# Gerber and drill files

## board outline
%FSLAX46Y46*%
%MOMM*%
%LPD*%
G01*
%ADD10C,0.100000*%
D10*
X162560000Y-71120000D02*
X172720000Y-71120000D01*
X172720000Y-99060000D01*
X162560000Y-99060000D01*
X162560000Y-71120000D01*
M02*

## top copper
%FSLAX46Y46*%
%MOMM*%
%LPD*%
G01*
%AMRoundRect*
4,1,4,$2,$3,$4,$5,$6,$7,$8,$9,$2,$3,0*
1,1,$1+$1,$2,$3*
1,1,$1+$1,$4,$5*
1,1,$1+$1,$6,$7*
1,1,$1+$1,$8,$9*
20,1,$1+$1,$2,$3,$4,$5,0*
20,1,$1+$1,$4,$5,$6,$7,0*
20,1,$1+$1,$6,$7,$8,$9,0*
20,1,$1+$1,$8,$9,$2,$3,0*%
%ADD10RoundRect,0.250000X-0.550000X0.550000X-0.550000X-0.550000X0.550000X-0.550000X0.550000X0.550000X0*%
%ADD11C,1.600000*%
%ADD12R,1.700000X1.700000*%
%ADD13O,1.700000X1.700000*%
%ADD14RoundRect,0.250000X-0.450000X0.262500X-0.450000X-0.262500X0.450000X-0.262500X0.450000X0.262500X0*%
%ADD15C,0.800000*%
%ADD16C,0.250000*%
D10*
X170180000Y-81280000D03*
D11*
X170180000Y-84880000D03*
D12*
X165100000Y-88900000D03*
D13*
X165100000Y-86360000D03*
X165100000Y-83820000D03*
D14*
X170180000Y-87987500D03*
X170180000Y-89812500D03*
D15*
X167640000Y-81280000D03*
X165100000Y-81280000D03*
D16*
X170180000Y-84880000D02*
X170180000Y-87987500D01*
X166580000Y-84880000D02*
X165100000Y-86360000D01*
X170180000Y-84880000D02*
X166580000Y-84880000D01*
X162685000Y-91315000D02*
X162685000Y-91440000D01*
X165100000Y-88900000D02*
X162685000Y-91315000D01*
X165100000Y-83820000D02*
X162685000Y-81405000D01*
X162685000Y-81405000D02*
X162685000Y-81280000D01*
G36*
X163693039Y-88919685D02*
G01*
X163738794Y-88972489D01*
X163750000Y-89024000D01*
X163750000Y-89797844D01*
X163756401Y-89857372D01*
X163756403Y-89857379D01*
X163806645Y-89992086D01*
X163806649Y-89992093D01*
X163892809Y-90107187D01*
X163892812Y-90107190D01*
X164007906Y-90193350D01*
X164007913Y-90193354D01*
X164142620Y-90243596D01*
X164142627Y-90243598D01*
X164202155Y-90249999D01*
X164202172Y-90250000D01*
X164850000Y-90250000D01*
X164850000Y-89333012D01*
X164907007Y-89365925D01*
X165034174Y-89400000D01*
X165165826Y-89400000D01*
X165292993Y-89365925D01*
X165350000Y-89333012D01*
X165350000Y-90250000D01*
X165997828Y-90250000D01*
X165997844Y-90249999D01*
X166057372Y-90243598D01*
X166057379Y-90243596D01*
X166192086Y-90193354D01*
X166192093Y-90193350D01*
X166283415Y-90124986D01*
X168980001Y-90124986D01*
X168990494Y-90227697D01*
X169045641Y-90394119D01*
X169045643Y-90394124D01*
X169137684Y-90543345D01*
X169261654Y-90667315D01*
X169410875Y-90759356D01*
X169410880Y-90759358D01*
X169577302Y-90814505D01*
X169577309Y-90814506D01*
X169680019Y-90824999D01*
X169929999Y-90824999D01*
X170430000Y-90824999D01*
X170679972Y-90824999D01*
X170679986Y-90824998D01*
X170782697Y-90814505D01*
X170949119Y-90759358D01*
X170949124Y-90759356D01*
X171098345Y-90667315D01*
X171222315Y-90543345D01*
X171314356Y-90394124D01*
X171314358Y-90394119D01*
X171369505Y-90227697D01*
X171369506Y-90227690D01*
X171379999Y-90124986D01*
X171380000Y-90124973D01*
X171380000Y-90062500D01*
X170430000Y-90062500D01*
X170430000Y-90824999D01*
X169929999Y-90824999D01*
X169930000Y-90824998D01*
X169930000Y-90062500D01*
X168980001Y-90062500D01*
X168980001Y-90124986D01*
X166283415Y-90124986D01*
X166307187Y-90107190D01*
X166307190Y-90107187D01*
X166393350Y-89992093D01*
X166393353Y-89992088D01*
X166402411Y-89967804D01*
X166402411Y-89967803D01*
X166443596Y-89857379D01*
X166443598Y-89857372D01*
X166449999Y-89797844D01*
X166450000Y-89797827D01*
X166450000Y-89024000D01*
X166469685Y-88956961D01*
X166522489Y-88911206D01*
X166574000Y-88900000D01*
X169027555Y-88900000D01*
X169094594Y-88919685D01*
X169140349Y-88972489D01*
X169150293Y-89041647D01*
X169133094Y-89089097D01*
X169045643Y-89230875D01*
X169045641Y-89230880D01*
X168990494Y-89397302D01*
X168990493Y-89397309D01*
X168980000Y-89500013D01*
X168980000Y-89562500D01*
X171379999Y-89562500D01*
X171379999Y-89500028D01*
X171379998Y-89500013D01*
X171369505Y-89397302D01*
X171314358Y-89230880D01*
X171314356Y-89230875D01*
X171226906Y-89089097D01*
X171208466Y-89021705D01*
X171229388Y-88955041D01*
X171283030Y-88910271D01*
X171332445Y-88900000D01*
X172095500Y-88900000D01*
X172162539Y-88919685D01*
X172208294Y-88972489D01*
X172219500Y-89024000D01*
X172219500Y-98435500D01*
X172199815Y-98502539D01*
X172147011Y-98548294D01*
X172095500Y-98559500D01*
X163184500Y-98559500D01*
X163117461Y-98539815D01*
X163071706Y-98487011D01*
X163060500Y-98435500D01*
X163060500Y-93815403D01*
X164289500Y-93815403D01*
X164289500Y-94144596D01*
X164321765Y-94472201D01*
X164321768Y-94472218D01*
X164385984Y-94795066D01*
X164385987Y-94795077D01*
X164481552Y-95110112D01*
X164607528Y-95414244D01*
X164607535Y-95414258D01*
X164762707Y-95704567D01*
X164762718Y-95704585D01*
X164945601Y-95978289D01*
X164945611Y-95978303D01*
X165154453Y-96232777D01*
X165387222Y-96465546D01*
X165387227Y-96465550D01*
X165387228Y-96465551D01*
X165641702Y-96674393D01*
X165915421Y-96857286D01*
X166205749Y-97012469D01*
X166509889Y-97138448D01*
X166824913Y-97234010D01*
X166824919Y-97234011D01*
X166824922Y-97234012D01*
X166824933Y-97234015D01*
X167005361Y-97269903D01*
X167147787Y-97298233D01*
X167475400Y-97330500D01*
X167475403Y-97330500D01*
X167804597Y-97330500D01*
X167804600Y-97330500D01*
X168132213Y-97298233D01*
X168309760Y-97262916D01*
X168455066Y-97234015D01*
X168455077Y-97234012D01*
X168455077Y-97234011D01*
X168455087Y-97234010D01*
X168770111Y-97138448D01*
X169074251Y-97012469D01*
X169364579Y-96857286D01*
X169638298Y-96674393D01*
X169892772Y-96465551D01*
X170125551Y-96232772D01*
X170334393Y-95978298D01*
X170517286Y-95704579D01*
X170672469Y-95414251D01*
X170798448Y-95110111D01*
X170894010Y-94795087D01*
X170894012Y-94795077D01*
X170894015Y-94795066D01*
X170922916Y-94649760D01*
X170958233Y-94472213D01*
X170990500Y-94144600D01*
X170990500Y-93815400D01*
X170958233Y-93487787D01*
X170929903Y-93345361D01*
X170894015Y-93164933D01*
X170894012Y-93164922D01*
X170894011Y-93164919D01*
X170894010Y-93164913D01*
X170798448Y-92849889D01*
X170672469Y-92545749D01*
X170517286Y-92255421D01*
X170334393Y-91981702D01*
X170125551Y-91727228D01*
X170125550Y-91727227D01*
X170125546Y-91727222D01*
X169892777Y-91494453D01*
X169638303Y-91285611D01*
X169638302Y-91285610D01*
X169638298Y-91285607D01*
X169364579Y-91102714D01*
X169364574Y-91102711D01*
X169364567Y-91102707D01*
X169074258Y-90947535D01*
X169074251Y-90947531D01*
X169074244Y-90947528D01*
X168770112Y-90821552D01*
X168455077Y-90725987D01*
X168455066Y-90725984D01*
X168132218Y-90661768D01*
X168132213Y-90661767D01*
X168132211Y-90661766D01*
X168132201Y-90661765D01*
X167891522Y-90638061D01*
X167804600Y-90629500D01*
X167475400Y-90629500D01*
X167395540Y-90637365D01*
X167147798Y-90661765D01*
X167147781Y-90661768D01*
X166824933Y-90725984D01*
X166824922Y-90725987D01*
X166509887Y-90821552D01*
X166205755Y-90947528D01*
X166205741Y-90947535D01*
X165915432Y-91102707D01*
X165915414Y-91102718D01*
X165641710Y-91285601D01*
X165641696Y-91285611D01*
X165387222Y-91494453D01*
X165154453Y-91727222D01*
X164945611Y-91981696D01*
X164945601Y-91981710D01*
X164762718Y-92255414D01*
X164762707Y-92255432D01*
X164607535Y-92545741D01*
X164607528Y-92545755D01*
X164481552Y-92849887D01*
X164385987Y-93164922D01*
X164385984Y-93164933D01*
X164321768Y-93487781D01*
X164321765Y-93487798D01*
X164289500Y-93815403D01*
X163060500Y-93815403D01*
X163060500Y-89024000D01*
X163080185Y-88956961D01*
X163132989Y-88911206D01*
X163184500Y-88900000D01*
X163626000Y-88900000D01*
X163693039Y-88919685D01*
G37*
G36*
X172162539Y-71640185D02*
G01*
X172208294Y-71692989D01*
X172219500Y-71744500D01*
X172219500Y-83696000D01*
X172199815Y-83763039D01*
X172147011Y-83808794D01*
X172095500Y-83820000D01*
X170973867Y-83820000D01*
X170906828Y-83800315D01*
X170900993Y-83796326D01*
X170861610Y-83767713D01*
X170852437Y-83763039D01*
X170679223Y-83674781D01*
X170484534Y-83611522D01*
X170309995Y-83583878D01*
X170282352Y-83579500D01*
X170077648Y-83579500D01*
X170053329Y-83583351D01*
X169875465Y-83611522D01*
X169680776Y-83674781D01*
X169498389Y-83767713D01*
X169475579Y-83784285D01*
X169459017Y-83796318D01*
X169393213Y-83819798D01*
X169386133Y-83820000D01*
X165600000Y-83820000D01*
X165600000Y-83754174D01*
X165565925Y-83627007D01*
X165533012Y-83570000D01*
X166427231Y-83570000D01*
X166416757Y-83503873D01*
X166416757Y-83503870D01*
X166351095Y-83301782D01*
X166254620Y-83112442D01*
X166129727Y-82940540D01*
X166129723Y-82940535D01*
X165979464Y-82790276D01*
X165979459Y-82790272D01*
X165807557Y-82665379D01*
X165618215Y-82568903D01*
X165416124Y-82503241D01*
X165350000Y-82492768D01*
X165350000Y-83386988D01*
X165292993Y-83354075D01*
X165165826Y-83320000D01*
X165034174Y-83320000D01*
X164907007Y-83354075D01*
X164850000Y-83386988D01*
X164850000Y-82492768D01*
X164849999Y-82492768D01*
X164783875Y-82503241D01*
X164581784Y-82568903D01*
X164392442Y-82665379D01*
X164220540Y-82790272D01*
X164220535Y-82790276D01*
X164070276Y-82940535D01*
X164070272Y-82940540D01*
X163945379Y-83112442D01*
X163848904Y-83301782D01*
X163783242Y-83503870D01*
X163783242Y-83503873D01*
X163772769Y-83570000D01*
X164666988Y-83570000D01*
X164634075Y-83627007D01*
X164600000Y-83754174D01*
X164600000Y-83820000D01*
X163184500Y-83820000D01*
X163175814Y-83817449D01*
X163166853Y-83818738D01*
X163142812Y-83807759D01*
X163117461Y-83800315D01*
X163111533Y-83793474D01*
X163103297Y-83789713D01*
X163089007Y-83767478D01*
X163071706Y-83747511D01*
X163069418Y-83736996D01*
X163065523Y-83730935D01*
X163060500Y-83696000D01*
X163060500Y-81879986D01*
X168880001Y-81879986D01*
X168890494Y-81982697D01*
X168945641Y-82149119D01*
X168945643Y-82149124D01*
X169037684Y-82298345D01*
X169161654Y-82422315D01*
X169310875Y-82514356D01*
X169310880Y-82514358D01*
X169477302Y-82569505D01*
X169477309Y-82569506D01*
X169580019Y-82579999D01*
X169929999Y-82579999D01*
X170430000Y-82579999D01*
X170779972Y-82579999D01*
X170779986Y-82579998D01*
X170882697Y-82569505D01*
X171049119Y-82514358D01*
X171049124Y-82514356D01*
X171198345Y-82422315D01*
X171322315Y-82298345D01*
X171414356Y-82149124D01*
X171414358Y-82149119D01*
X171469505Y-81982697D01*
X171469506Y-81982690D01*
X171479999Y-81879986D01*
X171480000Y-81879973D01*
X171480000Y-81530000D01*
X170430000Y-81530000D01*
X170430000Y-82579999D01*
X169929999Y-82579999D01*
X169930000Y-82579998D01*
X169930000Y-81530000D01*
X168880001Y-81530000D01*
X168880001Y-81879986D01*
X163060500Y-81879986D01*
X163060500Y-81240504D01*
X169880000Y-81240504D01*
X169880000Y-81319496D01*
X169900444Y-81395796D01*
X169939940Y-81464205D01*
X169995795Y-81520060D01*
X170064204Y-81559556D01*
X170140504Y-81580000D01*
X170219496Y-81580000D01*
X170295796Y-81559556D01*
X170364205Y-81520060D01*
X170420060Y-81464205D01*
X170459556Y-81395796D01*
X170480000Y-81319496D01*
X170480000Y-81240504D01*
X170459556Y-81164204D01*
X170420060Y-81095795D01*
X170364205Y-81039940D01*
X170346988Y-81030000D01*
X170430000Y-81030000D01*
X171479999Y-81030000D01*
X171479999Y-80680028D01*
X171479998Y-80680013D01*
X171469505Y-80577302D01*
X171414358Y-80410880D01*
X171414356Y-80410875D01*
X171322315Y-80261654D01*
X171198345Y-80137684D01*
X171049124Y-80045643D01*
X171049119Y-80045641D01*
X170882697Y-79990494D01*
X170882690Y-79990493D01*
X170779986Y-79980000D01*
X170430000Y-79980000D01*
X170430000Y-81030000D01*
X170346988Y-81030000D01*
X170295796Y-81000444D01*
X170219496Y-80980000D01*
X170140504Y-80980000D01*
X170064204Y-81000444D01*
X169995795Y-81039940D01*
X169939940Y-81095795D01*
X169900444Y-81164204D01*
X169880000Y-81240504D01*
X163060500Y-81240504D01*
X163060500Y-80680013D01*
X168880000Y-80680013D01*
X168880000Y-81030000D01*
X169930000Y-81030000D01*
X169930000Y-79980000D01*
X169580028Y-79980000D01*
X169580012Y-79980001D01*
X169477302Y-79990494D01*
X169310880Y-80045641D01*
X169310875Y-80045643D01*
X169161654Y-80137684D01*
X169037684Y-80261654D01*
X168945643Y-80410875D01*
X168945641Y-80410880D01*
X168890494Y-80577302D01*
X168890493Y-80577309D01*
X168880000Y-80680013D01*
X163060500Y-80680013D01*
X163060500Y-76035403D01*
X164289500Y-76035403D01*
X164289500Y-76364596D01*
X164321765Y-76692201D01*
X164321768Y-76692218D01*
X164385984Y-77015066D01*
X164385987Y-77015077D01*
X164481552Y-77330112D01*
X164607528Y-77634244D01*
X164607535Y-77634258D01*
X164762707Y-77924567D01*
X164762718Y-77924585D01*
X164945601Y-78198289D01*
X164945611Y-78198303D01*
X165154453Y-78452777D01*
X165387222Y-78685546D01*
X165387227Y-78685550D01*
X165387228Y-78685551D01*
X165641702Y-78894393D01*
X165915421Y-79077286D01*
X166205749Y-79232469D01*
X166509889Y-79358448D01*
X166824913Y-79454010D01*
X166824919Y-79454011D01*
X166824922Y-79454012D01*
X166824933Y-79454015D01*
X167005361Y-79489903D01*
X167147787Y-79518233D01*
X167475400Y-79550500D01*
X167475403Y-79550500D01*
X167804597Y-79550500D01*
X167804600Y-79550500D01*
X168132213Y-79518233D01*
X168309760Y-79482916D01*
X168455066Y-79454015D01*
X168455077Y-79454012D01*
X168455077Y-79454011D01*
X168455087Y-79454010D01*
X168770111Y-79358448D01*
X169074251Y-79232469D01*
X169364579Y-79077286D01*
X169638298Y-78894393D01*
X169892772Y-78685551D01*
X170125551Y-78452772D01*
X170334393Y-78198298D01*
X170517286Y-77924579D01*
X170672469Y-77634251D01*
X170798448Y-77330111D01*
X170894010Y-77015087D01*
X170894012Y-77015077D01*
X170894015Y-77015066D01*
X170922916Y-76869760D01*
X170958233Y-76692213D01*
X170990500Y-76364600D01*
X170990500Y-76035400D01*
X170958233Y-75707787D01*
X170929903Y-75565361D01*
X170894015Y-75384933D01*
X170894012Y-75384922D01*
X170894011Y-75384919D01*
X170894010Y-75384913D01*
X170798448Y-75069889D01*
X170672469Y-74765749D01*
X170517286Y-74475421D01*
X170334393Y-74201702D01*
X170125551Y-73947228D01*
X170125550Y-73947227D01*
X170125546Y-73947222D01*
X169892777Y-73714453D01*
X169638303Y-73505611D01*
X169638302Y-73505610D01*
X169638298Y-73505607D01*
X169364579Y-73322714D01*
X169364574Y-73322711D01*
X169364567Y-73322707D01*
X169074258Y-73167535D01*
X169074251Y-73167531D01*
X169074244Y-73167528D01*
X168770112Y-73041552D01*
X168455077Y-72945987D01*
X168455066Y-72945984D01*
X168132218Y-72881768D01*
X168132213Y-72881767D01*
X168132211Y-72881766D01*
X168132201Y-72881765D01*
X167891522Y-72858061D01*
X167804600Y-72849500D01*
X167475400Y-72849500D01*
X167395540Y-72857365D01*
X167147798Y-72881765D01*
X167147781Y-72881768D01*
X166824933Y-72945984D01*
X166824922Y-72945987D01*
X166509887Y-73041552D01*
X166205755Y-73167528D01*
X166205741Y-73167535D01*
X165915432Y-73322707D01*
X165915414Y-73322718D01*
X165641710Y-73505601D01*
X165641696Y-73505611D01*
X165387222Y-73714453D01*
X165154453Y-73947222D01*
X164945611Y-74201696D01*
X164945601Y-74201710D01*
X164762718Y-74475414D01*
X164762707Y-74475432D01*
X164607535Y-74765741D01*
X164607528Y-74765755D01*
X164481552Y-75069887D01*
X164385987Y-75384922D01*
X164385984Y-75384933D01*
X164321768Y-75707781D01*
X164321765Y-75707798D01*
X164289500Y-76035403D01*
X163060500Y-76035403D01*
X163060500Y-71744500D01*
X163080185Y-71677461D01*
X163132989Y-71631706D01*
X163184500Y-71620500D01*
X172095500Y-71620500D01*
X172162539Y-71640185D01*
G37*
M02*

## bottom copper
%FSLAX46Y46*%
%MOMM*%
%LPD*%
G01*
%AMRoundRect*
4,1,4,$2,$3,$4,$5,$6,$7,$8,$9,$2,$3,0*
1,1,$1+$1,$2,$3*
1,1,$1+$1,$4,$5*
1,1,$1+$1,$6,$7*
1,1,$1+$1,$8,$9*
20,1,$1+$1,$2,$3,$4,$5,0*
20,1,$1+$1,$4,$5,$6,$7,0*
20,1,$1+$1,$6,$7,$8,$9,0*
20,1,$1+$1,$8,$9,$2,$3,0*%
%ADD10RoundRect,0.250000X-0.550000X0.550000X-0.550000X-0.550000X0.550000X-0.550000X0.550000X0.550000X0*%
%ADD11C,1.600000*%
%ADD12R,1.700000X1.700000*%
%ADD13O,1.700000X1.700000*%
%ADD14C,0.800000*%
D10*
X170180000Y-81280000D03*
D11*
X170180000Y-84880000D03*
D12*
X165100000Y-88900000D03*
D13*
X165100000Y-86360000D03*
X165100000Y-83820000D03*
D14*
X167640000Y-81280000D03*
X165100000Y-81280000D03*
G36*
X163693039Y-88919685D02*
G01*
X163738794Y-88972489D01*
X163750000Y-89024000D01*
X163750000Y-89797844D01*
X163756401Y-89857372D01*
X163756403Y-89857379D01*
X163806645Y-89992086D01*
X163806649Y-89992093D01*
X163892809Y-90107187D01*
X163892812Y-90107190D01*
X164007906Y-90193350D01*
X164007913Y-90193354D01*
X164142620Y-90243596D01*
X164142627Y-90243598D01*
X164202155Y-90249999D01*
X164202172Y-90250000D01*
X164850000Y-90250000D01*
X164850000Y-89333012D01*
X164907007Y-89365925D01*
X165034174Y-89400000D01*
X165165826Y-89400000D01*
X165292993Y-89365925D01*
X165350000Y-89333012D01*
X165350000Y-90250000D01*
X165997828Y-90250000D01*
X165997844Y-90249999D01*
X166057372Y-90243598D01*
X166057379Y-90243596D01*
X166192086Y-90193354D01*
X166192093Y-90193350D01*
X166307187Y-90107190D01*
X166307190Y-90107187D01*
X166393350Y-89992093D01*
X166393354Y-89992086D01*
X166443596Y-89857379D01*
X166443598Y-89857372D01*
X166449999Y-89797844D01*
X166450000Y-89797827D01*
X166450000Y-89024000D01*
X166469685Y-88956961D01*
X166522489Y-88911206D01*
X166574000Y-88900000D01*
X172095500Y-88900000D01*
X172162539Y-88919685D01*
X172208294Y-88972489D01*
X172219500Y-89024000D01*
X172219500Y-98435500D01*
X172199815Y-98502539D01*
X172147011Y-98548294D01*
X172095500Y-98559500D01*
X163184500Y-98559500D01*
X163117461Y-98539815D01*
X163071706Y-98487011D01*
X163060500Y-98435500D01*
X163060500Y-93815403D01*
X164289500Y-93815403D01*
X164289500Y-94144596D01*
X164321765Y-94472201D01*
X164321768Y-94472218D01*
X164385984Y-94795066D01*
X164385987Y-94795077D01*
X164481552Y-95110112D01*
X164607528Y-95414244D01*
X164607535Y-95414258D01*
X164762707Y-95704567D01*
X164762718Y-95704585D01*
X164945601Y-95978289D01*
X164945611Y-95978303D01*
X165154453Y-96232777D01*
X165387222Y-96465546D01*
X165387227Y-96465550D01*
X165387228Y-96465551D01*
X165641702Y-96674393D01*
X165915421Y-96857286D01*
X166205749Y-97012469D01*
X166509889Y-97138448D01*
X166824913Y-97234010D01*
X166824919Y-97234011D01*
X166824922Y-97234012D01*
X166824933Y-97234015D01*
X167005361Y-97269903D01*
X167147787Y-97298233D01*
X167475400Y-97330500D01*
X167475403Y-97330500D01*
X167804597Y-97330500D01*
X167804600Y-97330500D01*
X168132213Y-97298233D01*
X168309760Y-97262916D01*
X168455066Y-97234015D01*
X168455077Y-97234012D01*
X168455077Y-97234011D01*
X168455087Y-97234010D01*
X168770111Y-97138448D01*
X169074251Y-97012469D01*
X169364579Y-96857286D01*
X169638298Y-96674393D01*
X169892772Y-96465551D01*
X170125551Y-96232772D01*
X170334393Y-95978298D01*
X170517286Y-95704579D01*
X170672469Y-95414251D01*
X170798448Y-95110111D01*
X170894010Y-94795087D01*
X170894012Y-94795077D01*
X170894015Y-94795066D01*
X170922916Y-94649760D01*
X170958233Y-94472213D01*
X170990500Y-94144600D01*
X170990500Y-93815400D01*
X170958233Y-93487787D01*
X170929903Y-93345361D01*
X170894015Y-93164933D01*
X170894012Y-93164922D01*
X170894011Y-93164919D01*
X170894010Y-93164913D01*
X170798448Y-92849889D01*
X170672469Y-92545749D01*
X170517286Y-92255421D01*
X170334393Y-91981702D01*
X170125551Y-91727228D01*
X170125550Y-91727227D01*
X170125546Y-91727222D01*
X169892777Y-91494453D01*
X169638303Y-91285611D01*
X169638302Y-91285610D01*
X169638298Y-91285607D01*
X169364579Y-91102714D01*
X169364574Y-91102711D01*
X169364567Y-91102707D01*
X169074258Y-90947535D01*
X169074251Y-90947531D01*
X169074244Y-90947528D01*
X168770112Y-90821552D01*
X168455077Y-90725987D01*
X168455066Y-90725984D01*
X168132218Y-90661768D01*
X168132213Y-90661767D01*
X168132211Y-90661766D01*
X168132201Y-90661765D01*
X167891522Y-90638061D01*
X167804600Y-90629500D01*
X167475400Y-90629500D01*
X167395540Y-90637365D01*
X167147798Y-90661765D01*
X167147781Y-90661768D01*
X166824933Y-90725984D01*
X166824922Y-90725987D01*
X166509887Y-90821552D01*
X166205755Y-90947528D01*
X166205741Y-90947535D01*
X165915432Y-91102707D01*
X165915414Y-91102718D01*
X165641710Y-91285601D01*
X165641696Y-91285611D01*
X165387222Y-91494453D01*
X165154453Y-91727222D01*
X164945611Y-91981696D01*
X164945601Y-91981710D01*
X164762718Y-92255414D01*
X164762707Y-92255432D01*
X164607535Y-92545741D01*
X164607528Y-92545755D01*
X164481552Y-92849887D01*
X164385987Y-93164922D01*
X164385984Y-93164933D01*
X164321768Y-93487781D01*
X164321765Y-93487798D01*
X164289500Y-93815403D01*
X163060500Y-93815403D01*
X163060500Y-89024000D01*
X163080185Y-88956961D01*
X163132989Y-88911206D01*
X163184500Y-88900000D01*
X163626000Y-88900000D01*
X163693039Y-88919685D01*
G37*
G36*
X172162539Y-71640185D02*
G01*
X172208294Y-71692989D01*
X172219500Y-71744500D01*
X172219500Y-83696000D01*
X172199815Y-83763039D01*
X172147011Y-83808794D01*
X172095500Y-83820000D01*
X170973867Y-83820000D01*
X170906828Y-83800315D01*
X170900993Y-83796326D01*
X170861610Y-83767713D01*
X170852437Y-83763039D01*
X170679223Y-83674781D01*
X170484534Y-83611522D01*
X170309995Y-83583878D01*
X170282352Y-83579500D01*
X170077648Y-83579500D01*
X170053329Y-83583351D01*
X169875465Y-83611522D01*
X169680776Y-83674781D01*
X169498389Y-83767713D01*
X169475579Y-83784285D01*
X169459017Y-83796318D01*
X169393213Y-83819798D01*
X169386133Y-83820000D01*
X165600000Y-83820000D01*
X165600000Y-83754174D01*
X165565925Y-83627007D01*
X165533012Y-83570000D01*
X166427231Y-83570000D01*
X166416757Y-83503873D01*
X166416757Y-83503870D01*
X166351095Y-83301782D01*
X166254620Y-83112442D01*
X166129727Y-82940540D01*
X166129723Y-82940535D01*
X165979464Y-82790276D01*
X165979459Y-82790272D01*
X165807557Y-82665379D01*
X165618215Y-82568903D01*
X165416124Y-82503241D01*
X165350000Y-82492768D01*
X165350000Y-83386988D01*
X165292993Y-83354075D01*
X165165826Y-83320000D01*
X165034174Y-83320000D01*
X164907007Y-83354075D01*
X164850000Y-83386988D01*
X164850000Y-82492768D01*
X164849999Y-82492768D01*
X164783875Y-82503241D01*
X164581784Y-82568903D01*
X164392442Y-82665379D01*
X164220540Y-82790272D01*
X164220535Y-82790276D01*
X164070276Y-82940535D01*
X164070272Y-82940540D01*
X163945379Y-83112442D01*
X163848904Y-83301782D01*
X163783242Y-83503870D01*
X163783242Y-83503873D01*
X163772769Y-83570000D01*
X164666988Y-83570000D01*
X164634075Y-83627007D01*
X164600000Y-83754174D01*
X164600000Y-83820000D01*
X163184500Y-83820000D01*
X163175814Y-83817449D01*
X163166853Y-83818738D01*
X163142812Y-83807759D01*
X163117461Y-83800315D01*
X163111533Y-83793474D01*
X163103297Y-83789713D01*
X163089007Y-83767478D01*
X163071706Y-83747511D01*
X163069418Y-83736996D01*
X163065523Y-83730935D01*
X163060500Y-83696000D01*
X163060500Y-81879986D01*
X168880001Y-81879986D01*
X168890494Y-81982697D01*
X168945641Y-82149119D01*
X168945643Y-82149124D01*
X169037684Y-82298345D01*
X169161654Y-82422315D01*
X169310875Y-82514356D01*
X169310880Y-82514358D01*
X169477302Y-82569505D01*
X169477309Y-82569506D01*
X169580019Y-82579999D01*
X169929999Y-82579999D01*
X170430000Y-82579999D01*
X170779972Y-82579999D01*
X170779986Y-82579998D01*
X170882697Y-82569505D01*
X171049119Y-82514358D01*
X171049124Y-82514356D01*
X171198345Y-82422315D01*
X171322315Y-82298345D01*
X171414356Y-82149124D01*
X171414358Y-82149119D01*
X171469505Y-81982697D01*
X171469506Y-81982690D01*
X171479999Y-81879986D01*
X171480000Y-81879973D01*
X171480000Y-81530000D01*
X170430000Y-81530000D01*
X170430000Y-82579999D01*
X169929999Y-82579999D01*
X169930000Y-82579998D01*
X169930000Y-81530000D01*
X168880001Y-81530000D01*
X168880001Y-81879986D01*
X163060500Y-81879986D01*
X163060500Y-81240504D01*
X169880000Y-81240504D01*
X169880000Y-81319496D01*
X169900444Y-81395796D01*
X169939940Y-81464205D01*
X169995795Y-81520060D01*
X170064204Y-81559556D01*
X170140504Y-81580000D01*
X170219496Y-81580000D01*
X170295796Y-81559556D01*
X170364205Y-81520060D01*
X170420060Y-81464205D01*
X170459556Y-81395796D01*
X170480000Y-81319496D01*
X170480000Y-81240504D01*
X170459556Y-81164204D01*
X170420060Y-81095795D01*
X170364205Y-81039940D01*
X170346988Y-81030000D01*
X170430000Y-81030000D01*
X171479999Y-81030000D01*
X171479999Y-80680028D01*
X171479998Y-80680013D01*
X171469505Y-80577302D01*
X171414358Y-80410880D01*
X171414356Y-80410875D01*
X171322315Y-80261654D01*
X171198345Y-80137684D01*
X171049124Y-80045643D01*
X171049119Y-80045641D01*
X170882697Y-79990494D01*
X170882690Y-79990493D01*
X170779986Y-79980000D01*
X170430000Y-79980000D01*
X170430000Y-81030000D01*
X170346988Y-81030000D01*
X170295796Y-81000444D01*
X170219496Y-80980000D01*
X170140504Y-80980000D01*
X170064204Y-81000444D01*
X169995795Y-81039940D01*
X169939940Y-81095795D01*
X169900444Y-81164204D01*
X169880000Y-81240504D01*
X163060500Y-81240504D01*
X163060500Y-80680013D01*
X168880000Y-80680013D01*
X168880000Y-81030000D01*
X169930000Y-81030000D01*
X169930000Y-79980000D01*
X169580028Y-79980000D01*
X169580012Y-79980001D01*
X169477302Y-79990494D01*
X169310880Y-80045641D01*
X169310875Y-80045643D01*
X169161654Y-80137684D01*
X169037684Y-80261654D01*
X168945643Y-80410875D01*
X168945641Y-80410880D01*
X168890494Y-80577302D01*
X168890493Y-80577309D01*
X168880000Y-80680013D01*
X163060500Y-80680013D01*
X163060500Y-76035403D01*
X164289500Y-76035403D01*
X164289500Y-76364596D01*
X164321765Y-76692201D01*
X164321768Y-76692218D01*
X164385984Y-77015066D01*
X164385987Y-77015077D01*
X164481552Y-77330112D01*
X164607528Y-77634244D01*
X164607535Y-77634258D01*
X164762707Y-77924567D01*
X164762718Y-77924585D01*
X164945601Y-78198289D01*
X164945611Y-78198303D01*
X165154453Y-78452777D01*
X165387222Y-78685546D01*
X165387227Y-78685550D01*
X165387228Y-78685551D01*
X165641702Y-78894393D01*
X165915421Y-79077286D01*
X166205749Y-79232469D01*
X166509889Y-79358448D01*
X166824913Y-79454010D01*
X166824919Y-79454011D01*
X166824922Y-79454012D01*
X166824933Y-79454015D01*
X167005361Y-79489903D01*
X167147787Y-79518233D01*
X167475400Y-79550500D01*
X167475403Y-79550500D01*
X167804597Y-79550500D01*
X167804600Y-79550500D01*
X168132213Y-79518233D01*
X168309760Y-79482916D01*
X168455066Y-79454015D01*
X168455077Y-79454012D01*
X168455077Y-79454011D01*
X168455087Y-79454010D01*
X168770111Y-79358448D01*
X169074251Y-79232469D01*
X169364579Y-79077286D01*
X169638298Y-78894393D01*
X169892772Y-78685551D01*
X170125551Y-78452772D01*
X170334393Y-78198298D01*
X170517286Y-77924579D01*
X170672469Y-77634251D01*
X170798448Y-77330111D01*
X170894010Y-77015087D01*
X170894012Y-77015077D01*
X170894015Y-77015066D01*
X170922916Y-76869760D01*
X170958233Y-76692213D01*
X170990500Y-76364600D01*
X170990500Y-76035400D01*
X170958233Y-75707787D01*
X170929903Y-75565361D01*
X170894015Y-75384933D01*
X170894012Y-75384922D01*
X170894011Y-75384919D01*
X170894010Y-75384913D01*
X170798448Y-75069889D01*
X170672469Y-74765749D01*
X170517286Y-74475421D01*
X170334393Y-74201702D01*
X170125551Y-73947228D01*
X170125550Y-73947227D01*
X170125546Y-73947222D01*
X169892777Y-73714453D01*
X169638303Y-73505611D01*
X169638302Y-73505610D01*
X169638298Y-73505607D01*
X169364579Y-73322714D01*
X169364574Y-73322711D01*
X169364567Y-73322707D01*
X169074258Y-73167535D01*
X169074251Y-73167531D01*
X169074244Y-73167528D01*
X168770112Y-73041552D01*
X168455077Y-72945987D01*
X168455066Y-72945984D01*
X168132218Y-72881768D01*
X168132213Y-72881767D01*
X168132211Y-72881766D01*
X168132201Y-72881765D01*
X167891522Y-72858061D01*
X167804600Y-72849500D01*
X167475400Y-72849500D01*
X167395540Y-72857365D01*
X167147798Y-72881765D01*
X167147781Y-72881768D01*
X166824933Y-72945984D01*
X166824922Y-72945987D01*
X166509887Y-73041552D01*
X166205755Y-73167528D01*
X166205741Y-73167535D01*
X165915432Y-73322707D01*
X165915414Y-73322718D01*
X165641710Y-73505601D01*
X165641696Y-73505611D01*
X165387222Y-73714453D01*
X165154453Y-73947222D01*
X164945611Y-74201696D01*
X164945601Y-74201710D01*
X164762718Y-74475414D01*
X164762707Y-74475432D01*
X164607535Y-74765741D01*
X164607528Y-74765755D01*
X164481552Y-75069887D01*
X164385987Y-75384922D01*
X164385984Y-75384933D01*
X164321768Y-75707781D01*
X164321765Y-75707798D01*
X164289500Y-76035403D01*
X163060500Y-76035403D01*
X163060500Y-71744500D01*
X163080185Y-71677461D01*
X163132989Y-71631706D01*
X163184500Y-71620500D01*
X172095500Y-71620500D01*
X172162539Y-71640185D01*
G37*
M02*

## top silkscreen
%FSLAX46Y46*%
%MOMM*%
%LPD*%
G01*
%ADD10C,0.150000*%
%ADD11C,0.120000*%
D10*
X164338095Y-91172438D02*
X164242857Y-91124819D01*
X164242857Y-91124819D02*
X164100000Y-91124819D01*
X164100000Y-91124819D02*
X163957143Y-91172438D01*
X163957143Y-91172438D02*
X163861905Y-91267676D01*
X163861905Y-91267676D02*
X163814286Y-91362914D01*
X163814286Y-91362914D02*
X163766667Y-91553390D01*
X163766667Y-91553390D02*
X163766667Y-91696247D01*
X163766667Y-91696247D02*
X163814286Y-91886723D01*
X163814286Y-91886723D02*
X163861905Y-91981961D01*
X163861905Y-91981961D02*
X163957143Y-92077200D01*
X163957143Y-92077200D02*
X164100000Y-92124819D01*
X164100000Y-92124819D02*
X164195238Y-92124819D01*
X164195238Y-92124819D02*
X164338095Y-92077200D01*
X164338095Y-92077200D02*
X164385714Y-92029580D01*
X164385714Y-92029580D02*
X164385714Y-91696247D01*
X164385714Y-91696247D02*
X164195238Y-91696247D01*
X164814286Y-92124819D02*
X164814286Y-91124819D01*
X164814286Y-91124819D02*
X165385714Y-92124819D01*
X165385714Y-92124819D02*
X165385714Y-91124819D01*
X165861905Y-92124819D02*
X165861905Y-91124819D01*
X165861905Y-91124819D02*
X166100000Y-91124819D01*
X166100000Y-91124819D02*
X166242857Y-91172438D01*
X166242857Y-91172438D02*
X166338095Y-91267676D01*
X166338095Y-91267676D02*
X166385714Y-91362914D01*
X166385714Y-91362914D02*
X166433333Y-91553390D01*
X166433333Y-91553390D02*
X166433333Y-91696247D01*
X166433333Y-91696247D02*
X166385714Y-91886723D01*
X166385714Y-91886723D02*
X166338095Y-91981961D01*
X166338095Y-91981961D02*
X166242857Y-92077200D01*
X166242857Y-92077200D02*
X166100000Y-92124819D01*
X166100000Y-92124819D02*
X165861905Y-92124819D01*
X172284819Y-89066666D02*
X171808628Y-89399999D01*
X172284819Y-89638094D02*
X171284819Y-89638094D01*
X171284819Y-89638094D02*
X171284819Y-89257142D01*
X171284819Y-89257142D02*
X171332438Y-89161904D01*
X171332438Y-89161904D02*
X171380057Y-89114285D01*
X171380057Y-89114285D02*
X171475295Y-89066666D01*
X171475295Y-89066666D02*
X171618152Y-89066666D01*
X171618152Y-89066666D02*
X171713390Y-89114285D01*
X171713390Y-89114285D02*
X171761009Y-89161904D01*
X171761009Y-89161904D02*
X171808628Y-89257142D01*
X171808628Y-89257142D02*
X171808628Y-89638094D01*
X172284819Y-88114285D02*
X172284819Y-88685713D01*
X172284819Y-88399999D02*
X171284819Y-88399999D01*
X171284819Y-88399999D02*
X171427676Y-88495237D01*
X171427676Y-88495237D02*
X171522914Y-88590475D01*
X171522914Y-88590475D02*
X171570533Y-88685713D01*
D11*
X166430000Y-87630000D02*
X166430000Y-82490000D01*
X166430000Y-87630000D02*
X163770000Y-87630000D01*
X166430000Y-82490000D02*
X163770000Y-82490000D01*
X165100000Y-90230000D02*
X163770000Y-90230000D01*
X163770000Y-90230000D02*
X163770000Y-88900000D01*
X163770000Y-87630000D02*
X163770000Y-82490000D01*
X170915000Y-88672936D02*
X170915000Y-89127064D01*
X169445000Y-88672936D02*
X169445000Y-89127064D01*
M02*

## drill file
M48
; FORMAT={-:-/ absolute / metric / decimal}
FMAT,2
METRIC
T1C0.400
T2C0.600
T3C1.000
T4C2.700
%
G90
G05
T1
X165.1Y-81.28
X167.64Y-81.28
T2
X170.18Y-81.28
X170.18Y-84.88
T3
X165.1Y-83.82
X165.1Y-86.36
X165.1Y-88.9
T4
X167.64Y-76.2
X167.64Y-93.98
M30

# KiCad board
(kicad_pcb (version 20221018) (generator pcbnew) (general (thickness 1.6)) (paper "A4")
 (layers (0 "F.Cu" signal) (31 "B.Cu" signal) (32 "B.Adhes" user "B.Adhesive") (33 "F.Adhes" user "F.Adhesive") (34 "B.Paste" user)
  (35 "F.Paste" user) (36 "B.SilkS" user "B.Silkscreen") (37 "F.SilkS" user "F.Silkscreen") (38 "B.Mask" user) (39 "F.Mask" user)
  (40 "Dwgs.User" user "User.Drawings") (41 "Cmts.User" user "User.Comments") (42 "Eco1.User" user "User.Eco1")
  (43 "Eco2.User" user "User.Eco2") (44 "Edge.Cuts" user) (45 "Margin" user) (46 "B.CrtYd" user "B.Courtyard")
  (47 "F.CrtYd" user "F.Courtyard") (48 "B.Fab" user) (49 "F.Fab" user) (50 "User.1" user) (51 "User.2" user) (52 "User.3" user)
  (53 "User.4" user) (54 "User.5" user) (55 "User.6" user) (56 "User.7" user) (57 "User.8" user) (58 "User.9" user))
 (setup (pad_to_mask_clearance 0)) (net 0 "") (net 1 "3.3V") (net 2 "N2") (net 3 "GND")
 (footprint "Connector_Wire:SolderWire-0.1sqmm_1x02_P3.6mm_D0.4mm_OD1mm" (layer "F.Cu") (at 170.18 81.28 -90)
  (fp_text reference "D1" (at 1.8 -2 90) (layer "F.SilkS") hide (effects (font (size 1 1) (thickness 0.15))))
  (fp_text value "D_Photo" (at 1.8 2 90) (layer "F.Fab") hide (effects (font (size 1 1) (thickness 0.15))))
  (pad "1" thru_hole roundrect (at 0 0 270) (size 1.6 1.6) (drill 0.6) (layers "*.Cu" "*.Mask") (roundrect_rratio 0.15625) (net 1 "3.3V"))
  (pad "2" thru_hole circle (at 3.6 0 270) (size 1.6 1.6) (drill 0.6) (layers "*.Cu" "*.Mask") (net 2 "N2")))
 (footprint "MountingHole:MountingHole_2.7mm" (layer "F.Cu") (at 167.64 93.98)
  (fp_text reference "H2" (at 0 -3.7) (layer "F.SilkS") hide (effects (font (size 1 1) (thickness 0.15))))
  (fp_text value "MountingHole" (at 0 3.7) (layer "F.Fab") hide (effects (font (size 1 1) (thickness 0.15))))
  (pad "" np_thru_hole circle (at 0 0) (size 2.7 2.7) (drill 2.7) (layers "F&B.Cu" "*.Mask") (clearance 2)))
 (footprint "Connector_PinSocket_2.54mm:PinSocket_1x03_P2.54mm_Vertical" (layer "F.Cu") (at 165.1 88.9 180)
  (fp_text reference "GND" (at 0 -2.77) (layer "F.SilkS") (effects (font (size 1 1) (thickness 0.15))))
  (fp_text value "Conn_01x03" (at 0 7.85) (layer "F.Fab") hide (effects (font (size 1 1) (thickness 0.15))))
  (fp_line (start -1.33 1.27) (end -1.33 6.41) (stroke (width 0.12) (type solid)) (layer "F.SilkS"))
  (fp_line (start -1.33 1.27) (end 1.33 1.27) (stroke (width 0.12) (type solid)) (layer "F.SilkS"))
  (fp_line (start -1.33 6.41) (end 1.33 6.41) (stroke (width 0.12) (type solid)) (layer "F.SilkS"))
  (fp_line (start 0 -1.33) (end 1.33 -1.33) (stroke (width 0.12) (type solid)) (layer "F.SilkS"))
  (fp_line (start 1.33 -1.33) (end 1.33 0) (stroke (width 0.12) (type solid)) (layer "F.SilkS"))
  (fp_line (start 1.33 1.27) (end 1.33 6.41) (stroke (width 0.12) (type solid)) (layer "F.SilkS"))
  (pad "1" thru_hole rect (at 0 0 180) (size 1.7 1.7) (drill 1) (layers "*.Cu" "*.Mask") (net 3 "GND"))
  (pad "2" thru_hole oval (at 0 2.54 180) (size 1.7 1.7) (drill 1) (layers "*.Cu" "*.Mask") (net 2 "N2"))
  (pad "3" thru_hole oval (at 0 5.08 180) (size 1.7 1.7) (drill 1) (layers "*.Cu" "*.Mask") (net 1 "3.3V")))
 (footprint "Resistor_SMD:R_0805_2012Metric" (layer "F.Cu") (at 170.18 88.9 -90)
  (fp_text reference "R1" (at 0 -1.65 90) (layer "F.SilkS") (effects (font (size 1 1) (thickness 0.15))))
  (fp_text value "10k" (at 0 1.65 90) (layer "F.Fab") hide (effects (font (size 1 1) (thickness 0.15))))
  (fp_line (start -0.227064 -0.735) (end 0.227064 -0.735) (stroke (width 0.12) (type solid)) (layer "F.SilkS"))
  (fp_line (start -0.227064 0.735) (end 0.227064 0.735) (stroke (width 0.12) (type solid)) (layer "F.SilkS"))
  (pad "1" smd roundrect (at -0.9125 0 270) (size 1.025 1.4) (layers "F.Cu" "F.Paste" "F.Mask") (roundrect_rratio 0.243902) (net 2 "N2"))
  (pad "2" smd roundrect (at 0.9125 0 270) (size 1.025 1.4) (layers "F.Cu" "F.Paste" "F.Mask") (roundrect_rratio 0.243902) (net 3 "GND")))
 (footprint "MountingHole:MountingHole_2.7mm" (layer "F.Cu") (at 167.64 76.2)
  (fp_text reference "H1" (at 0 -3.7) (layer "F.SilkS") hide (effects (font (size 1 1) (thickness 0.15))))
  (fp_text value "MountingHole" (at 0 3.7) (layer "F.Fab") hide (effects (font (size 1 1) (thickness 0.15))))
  (pad "" np_thru_hole circle (at 0 0) (size 2.7 2.7) (drill 2.7) (layers "F&B.Cu" "*.Mask") (clearance 2)))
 (gr_rect (start 162.56 71.12) (end 172.72 99.06) (stroke (width 0.1) (type default)) (fill none) (layer "Edge.Cuts"))
 (segment (start 170.18 84.88) (end 170.18 87.9875) (width 0.25) (layer "F.Cu") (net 2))
 (segment (start 166.58 84.88) (end 165.1 86.36) (width 0.25) (layer "F.Cu") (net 2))
 (segment (start 170.18 84.88) (end 166.58 84.88) (width 0.25) (layer "F.Cu") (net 2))
 (segment (start 162.685 91.315) (end 162.685 91.44) (width 0.25) (layer "F.Cu") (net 3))
 (segment (start 165.1 88.9) (end 162.685 91.315) (width 0.25) (layer "F.Cu") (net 3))
 (segment (start 165.1 83.82) (end 162.685 81.405) (width 0.25) (layer "F.Cu") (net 1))
 (segment (start 162.685 81.405) (end 162.685 81.28) (width 0.25) (layer "F.Cu") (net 1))
 (via (at 167.64 81.28) (size 0.8) (drill 0.4) (layers "F.Cu" "B.Cu") (free) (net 1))
 (via (at 165.1 81.28) (size 0.8) (drill 0.4) (layers "F.Cu" "B.Cu") (free) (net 1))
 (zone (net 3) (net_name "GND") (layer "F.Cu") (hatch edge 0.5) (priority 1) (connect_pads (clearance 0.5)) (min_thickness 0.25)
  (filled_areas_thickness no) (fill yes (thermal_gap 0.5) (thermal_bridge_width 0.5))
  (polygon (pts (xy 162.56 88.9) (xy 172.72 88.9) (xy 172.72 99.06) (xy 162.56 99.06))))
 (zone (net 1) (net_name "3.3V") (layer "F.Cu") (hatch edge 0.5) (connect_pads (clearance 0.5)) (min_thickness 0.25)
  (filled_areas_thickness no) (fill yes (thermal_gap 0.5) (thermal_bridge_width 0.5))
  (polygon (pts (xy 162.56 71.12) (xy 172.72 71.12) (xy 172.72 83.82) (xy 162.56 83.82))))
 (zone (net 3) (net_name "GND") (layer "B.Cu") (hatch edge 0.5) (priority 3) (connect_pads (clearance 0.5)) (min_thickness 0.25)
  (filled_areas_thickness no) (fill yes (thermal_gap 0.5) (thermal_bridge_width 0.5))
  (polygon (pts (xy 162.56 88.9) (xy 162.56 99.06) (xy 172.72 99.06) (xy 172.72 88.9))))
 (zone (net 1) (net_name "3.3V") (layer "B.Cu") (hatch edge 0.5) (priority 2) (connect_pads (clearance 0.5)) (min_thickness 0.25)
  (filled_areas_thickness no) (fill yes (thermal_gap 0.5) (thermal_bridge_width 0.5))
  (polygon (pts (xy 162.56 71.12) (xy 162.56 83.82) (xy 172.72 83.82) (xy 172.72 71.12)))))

